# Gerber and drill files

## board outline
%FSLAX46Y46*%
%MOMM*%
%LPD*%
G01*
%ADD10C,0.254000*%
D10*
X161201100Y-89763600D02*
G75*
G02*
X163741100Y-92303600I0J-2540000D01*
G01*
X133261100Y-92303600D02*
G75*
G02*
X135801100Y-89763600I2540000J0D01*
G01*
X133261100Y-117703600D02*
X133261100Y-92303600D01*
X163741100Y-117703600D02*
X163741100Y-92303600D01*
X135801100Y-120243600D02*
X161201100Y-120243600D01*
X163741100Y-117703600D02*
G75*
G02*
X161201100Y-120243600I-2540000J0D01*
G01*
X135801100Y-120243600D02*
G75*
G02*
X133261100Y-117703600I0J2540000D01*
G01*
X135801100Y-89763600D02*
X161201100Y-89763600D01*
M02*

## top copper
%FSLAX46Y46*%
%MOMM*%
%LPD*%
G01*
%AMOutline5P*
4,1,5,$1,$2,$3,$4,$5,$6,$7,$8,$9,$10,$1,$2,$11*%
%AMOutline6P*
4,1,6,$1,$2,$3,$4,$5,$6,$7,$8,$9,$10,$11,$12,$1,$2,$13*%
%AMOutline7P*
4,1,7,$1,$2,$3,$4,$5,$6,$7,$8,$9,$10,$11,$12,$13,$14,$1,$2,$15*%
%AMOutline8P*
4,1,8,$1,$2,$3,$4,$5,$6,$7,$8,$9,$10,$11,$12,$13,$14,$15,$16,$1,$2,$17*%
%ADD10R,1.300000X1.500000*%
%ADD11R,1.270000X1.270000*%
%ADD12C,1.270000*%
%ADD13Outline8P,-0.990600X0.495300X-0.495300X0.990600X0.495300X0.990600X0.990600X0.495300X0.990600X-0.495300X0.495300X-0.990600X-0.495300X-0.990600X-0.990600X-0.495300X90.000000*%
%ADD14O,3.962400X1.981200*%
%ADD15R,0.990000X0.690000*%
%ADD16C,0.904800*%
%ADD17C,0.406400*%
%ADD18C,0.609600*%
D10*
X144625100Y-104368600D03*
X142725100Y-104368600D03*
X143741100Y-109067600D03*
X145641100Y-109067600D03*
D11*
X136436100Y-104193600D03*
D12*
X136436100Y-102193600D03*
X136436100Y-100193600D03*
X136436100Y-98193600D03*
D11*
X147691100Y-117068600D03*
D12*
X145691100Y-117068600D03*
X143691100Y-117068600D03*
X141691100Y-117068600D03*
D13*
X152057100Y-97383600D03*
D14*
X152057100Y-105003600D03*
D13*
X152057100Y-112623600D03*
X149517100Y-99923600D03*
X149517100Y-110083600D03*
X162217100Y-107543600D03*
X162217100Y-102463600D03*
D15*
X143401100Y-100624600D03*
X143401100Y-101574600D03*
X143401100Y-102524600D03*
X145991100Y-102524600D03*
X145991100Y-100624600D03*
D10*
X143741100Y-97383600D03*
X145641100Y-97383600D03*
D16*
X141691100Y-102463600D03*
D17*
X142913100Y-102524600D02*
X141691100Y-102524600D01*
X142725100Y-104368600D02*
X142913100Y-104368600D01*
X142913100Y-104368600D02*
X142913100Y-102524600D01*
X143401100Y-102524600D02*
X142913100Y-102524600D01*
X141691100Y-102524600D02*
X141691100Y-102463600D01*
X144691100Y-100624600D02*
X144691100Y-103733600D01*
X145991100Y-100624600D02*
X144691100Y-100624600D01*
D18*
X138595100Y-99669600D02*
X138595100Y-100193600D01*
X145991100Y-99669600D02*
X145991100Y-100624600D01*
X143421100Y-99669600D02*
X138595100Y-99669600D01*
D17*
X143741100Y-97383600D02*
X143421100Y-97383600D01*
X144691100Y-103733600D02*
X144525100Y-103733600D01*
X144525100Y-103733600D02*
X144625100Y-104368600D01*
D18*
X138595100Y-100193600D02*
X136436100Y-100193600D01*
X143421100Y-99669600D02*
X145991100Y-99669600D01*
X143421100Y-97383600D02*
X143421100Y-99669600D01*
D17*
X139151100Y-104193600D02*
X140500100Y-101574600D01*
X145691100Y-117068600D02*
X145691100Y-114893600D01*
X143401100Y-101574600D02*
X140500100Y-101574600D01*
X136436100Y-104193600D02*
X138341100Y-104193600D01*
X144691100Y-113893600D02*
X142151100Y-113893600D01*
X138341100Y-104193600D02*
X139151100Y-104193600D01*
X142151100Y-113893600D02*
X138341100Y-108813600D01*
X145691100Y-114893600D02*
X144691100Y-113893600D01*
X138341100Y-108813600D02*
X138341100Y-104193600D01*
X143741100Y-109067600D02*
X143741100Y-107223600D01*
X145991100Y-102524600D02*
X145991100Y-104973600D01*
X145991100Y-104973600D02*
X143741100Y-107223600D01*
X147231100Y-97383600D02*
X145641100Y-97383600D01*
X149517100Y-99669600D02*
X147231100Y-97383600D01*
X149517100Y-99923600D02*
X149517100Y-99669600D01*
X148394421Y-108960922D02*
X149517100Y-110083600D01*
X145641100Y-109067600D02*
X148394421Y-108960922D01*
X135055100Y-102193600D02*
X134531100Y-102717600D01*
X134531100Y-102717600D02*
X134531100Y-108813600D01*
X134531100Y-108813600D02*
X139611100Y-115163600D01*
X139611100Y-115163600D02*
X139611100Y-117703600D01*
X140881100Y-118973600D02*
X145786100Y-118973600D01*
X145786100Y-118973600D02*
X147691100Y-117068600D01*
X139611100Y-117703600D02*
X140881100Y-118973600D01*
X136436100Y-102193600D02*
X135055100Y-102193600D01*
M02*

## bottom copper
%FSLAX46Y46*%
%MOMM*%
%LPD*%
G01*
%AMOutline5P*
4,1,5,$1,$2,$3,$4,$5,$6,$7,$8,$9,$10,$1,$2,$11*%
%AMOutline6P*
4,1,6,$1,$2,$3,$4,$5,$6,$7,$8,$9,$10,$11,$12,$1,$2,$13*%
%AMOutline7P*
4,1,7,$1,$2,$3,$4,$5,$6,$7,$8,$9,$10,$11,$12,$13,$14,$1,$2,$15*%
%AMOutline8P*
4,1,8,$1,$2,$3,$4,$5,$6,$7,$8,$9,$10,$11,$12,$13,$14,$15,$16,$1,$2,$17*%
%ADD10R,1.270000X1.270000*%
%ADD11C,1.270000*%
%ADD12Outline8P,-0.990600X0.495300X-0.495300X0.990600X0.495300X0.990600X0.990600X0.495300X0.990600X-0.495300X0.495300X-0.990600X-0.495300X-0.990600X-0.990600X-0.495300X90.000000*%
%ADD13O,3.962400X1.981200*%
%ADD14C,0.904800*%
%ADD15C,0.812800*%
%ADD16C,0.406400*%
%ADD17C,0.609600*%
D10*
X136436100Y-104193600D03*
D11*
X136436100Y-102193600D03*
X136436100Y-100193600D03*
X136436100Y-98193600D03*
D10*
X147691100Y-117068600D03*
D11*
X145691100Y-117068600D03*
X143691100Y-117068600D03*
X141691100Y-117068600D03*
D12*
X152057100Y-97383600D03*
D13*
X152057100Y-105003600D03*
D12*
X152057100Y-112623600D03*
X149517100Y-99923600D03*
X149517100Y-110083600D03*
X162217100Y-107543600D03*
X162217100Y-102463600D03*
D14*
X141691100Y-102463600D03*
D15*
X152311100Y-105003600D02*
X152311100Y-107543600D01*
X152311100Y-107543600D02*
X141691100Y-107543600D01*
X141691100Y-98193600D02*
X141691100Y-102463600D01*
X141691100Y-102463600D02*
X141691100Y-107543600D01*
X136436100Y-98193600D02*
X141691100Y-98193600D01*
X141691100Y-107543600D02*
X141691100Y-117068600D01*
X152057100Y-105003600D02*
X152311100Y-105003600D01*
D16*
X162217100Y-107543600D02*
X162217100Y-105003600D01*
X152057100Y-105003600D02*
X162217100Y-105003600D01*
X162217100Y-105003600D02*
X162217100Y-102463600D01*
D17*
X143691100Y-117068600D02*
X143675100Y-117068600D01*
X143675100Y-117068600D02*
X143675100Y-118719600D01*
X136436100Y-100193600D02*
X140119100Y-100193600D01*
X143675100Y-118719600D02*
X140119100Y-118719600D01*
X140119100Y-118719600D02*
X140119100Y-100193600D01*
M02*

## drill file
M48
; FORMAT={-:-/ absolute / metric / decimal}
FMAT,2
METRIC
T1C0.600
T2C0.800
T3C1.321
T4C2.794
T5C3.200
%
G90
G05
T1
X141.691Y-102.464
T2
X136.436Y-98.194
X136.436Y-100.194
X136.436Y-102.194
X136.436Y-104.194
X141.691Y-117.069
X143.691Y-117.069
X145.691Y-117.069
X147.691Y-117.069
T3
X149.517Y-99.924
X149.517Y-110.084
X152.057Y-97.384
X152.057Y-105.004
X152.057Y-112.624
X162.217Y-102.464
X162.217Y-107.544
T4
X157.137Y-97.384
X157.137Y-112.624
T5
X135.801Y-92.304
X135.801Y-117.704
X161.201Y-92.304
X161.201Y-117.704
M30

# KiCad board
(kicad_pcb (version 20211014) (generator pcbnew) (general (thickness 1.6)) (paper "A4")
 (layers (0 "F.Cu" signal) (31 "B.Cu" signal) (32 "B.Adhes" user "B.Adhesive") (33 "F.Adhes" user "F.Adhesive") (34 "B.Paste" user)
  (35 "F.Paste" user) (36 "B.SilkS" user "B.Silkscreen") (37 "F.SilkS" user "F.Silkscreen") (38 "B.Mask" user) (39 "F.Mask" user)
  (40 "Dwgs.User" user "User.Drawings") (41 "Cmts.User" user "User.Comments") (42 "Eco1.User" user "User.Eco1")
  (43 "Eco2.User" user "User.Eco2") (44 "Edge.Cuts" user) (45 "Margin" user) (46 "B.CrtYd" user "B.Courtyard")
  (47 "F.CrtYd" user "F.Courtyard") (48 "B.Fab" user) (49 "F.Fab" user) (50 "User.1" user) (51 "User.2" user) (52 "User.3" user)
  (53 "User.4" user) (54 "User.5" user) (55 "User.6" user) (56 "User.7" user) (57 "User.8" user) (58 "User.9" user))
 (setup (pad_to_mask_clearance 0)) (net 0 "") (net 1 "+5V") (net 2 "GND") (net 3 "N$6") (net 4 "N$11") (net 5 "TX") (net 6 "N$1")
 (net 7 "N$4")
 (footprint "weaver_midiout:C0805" (layer "F.Cu") (at 143.6751 104.3686 180)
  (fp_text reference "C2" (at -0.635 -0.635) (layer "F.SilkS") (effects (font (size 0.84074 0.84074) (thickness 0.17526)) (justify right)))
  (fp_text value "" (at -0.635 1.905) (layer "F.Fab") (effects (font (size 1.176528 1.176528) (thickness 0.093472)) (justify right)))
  (pad "1" smd rect (at -0.95 0 180) (size 1.3 1.5) (layers "F.Cu" "F.Paste" "F.Mask") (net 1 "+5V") (solder_mask_margin 0.0508))
  (pad "2" smd rect (at 0.95 0 180) (size 1.3 1.5) (layers "F.Cu" "F.Paste" "F.Mask") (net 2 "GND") (solder_mask_margin 0.0508)))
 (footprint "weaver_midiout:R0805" (layer "F.Cu") (at 144.6911 109.0676)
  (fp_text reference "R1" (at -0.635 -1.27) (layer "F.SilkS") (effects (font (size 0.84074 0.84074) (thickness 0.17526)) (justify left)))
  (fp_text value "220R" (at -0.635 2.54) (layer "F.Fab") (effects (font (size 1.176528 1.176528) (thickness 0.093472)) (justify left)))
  (pad "1" smd rect (at -0.95 0) (size 1.3 1.5) (layers "F.Cu" "F.Paste" "F.Mask") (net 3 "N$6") (solder_mask_margin 0.0508))
  (pad "2" smd rect (at 0.95 0) (size 1.3 1.5) (layers "F.Cu" "F.Paste" "F.Mask") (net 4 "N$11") (solder_mask_margin 0.0508)))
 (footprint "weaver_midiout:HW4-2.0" (layer "F.Cu") (at 136.4361 101.1936 90)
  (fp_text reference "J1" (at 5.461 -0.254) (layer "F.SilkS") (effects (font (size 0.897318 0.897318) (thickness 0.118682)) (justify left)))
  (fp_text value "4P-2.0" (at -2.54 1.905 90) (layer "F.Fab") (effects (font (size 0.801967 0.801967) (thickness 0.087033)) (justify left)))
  (pad "1" thru_hole rect (at -3 0 90) (size 1.27 1.27) (drill 0.8) (layers *.Cu *.Mask) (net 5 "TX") (solder_mask_margin 0.0508))
  (pad "2" thru_hole circle (at -1 0 90) (size 1.27 1.27) (drill 0.8) (layers *.Cu *.Mask) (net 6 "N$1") (solder_mask_margin 0.0508))
  (pad "3" thru_hole circle (at 1 0 90) (size 1.27 1.27) (drill 0.8) (layers *.Cu *.Mask) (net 1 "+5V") (solder_mask_margin 0.0508))
  (pad "4" thru_hole circle (at 3 0 90) (size 1.27 1.27) (drill 0.8) (layers *.Cu *.Mask) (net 2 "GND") (solder_mask_margin 0.0508)))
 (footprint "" (layer "F.Cu") (at 161.2011 92.3036)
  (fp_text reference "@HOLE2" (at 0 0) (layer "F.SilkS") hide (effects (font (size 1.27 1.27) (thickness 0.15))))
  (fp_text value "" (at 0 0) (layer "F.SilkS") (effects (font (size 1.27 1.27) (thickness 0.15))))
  (pad "" np_thru_hole circle (at 0 0) (size 3.2 3.2) (drill 3.2) (layers *.Cu *.Mask)))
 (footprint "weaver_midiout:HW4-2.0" (layer "F.Cu") (at 144.6911 117.0686 180)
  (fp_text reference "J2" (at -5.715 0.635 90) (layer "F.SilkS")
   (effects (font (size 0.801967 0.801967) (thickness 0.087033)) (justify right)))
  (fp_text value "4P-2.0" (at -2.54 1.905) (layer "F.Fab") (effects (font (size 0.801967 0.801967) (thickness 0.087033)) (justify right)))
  (pad "1" thru_hole rect (at -3 0 180) (size 1.27 1.27) (drill 0.8) (layers *.Cu *.Mask) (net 6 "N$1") (solder_mask_margin 0.0508))
  (pad "2" thru_hole circle (at -1 0 180) (size 1.27 1.27) (drill 0.8) (layers *.Cu *.Mask) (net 5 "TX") (solder_mask_margin 0.0508))
  (pad "3" thru_hole circle (at 1 0 180) (size 1.27 1.27) (drill 0.8) (layers *.Cu *.Mask) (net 1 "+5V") (solder_mask_margin 0.0508))
  (pad "4" thru_hole circle (at 3 0 180) (size 1.27 1.27) (drill 0.8) (layers *.Cu *.Mask) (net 2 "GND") (solder_mask_margin 0.0508)))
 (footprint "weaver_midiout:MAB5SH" (layer "F.Cu") (at 157.1371 105.0036 90)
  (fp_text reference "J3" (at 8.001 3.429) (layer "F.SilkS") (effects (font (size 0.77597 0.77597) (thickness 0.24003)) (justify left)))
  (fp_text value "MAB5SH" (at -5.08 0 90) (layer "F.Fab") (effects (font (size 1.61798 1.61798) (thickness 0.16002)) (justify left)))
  (pad "" np_thru_hole circle (at -7.62 0 90) (size 2.794 2.794) (drill 2.794) (layers *.Cu *.Mask))
  (pad "" np_thru_hole circle (at 7.62 0 90) (size 2.794 2.794) (drill 2.794) (layers *.Cu *.Mask))
  (pad "1" thru_hole roundrect (at 7.62 -5.08 90) (size 1.9812 1.9812) (drill 1.3208) (layers *.Cu *.Mask) (roundrect_rratio 0.25)
   (chamfer_ratio 0.25) (chamfer top_left top_right bottom_left bottom_right) (solder_mask_margin 0.0508))
  (pad "2" thru_hole oval (at 0 -5.08 180) (size 3.9624 1.9812) (drill 1.3208) (layers *.Cu *.Mask) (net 2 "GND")
   (solder_mask_margin 0.0508))
  (pad "3" thru_hole roundrect (at -7.62 -5.08 90) (size 1.9812 1.9812) (drill 1.3208) (layers *.Cu *.Mask) (roundrect_rratio 0.25)
   (chamfer_ratio 0.25) (chamfer top_left top_right bottom_left bottom_right) (solder_mask_margin 0.0508))
  (pad "4" thru_hole roundrect (at 5.08 -7.62 90) (size 1.9812 1.9812) (drill 1.3208) (layers *.Cu *.Mask) (roundrect_rratio 0.25)
   (chamfer_ratio 0.25) (chamfer top_left top_right bottom_left bottom_right) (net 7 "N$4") (solder_mask_margin 0.0508))
  (pad "5" thru_hole roundrect (at -5.08 -7.62 90) (size 1.9812 1.9812) (drill 1.3208) (layers *.Cu *.Mask) (roundrect_rratio 0.25)
   (chamfer_ratio 0.25) (chamfer top_left top_right bottom_left bottom_right) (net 4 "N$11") (solder_mask_margin 0.0508))
  (pad "PE" thru_hole roundrect (at -2.54 5.08 90) (size 1.9812 1.9812) (drill 1.3208) (layers *.Cu *.Mask) (roundrect_rratio 0.25)
   (chamfer_ratio 0.25) (chamfer top_left top_right bottom_left bottom_right) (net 2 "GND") (solder_mask_margin 0.0508))
  (pad "PE@" thru_hole roundrect (at 2.54 5.08 90) (size 1.9812 1.9812) (drill 1.3208) (layers *.Cu *.Mask) (roundrect_rratio 0.25)
   (chamfer_ratio 0.25) (chamfer top_left top_right bottom_left bottom_right) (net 2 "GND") (solder_mask_margin 0.0508)))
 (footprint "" (layer "F.Cu") (at 161.2011 117.7036)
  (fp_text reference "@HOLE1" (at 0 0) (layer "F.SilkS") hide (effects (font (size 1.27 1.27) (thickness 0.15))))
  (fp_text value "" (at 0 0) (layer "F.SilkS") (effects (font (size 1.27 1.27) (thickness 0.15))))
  (pad "" np_thru_hole circle (at 0 0) (size 3.2 3.2) (drill 3.2) (layers *.Cu *.Mask)))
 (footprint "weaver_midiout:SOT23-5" (layer "F.Cu") (at 144.6911 101.5746 -90)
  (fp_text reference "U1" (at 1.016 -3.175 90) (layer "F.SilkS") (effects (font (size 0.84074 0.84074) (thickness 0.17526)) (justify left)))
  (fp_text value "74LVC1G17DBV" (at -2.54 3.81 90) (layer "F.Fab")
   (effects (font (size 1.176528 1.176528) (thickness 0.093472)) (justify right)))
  (pad "1" smd rect (at -0.95 1.29 270) (size 0.69 0.99) (layers "F.Cu" "F.Paste" "F.Mask") (solder_mask_margin 0.0508))
  (pad "2" smd rect (at 0 1.29 270) (size 0.69 0.99) (layers "F.Cu" "F.Paste" "F.Mask") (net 5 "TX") (solder_mask_margin 0.0508))
  (pad "3" smd rect (at 0.95 1.29 270) (size 0.69 0.99) (layers "F.Cu" "F.Paste" "F.Mask") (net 2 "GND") (solder_mask_margin 0.0508))
  (pad "4" smd rect (at 0.95 -1.3 270) (size 0.69 0.99) (layers "F.Cu" "F.Paste" "F.Mask") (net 3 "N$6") (solder_mask_margin 0.0508))
  (pad "5" smd rect (at -0.95 -1.3 270) (size 0.69 0.99) (layers "F.Cu" "F.Paste" "F.Mask") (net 1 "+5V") (solder_mask_margin 0.0508)))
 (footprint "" (layer "F.Cu") (at 135.8011 117.7036)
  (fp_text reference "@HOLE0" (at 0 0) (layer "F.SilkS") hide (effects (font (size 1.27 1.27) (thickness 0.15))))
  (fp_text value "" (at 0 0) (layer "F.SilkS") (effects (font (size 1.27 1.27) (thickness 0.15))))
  (pad "" np_thru_hole circle (at 0 0) (size 3.2 3.2) (drill 3.2) (layers *.Cu *.Mask)))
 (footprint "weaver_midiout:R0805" (layer "F.Cu") (at 144.6911 97.3836)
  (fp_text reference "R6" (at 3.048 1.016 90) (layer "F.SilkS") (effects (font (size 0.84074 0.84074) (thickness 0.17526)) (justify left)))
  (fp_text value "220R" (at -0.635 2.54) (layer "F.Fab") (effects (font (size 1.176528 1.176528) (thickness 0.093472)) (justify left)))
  (pad "1" smd rect (at -0.95 0) (size 1.3 1.5) (layers "F.Cu" "F.Paste" "F.Mask") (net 1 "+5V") (solder_mask_margin 0.0508))
  (pad "2" smd rect (at 0.95 0) (size 1.3 1.5) (layers "F.Cu" "F.Paste" "F.Mask") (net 7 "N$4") (solder_mask_margin 0.0508)))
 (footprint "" (layer "F.Cu") (at 135.8011 92.3036)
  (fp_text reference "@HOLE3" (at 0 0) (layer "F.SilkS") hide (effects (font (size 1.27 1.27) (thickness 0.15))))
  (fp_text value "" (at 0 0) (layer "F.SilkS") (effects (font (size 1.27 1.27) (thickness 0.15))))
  (pad "" np_thru_hole circle (at 0 0) (size 3.2 3.2) (drill 3.2) (layers *.Cu *.Mask)))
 (gr_arc (start 161.2011 89.7636) (mid 162.997151 90.507549) (end 163.7411 92.3036) (layer "Edge.Cuts") (width 0.254))
 (gr_arc (start 133.2611 92.3036) (mid 134.005049 90.507549) (end 135.8011 89.7636) (layer "Edge.Cuts") (width 0.254))
 (gr_line (start 133.2611 117.7036) (end 133.2611 92.3036) (layer "Edge.Cuts") (width 0.254))
 (gr_line (start 163.7411 117.7036) (end 163.7411 92.3036) (layer "Edge.Cuts") (width 0.254))
 (gr_line (start 135.8011 120.2436) (end 161.2011 120.2436) (layer "Edge.Cuts") (width 0.254))
 (gr_arc (start 163.7411 117.7036) (mid 162.997151 119.499651) (end 161.2011 120.2436) (layer "Edge.Cuts") (width 0.254))
 (gr_arc (start 135.8011 120.2436) (mid 134.005049 119.499651) (end 133.2611 117.7036) (layer "Edge.Cuts") (width 0.254))
 (gr_line (start 135.8011 89.7636) (end 161.2011 89.7636) (layer "Edge.Cuts") (width 0.254))
 (segment (start 142.9131 102.5246) (end 141.6911 102.5246) (width 0.4064) (layer "F.Cu") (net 2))
 (segment (start 142.7251 104.3686) (end 142.9131 104.3686) (width 0.4064) (layer "F.Cu") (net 2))
 (segment (start 142.9131 104.3686) (end 142.9131 102.5246) (width 0.4064) (layer "F.Cu") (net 2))
 (segment (start 143.4011 102.5246) (end 142.9131 102.5246) (width 0.4064) (layer "F.Cu") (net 2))
 (segment (start 141.6911 102.5246) (end 141.6911 102.4636) (width 0.4064) (layer "F.Cu") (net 2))
 (via (at 141.6911 102.4636) (size 0.9048) (drill 0.6) (layers "F.Cu" "B.Cu") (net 2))
 (segment (start 152.3111 105.0036) (end 152.3111 107.5436) (width 0.8128) (layer "B.Cu") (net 2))
 (segment (start 152.3111 107.5436) (end 141.6911 107.5436) (width 0.8128) (layer "B.Cu") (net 2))
 (segment (start 141.6911 98.1936) (end 141.6911 102.4636) (width 0.8128) (layer "B.Cu") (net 2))
 (segment (start 141.6911 102.4636) (end 141.6911 107.5436) (width 0.8128) (layer "B.Cu") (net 2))
 (segment (start 136.4361 98.1936) (end 141.6911 98.1936) (width 0.8128) (layer "B.Cu") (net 2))
 (segment (start 141.6911 107.5436) (end 141.6911 117.0686) (width 0.8128) (layer "B.Cu") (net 2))
 (segment (start 152.0571 105.0036) (end 152.3111 105.0036) (width 0.8128) (layer "B.Cu") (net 2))
 (segment (start 162.2171 107.5436) (end 162.2171 105.0036) (width 0.4064) (layer "B.Cu") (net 2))
 (segment (start 152.0571 105.0036) (end 162.2171 105.0036) (width 0.4064) (layer "B.Cu") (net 2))
 (segment (start 162.2171 105.0036) (end 162.2171 102.4636) (width 0.4064) (layer "B.Cu") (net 2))
 (segment (start 144.6911 100.6246) (end 144.6911 103.7336) (width 0.4064) (layer "F.Cu") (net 1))
 (segment (start 145.9911 100.6246) (end 144.6911 100.6246) (width 0.4064) (layer "F.Cu") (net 1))
 (segment (start 138.5951 99.6696) (end 138.5951 100.1936) (width 0.6096) (layer "F.Cu") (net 1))
 (segment (start 145.9911 99.6696) (end 145.9911 100.6246) (width 0.6096) (layer "F.Cu") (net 1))
 (segment (start 143.4211 99.6696) (end 138.5951 99.6696) (width 0.6096) (layer "F.Cu") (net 1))
 (segment (start 143.7411 97.3836) (end 143.4211 97.3836) (width 0.4064) (layer "F.Cu") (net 1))
 (segment (start 144.6911 103.7336) (end 144.5251 103.7336) (width 0.4064) (layer "F.Cu") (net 1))
 (segment (start 144.5251 103.7336) (end 144.6251 104.3686) (width 0.4064) (layer "F.Cu") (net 1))
 (segment (start 138.5951 100.1936) (end 136.4361 100.1936) (width 0.6096) (layer "F.Cu") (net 1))
 (segment (start 143.4211 99.6696) (end 145.9911 99.6696) (width 0.6096) (layer "F.Cu") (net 1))
 (segment (start 143.4211 97.3836) (end 143.4211 99.6696) (width 0.6096) (layer "F.Cu") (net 1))
 (segment (start 143.6911 117.0686) (end 143.6751 117.0686) (width 0.6096) (layer "B.Cu") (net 1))
 (segment (start 143.6751 117.0686) (end 143.6751 118.7196) (width 0.6096) (layer "B.Cu") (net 1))
 (segment (start 136.4361 100.1936) (end 140.1191 100.1936) (width 0.6096) (layer "B.Cu") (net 1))
 (segment (start 143.6751 118.7196) (end 140.1191 118.7196) (width 0.6096) (layer "B.Cu") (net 1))
 (segment (start 140.1191 118.7196) (end 140.1191 100.1936) (width 0.6096) (layer "B.Cu") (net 1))
 (segment (start 139.1511 104.1936) (end 140.5001 101.5746) (width 0.4064) (layer "F.Cu") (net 5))
 (segment (start 145.6911 117.0686) (end 145.6911 114.8936) (width 0.4064) (layer "F.Cu") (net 5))
 (segment (start 143.4011 101.5746) (end 140.5001 101.5746) (width 0.4064) (layer "F.Cu") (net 5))
 (segment (start 136.4361 104.1936) (end 138.3411 104.1936) (width 0.4064) (layer "F.Cu") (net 5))
 (segment (start 144.6911 113.8936) (end 142.1511 113.8936) (width 0.4064) (layer "F.Cu") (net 5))
 (segment (start 138.3411 104.1936) (end 139.1511 104.1936) (width 0.4064) (layer "F.Cu") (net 5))
 (segment (start 142.1511 113.8936) (end 138.3411 108.8136) (width 0.4064) (layer "F.Cu") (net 5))
 (segment (start 145.6911 114.8936) (end 144.6911 113.8936) (width 0.4064) (layer "F.Cu") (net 5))
 (segment (start 138.3411 108.8136) (end 138.3411 104.1936) (width 0.4064) (layer "F.Cu") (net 5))
 (segment (start 143.7411 109.0676) (end 143.7411 107.2236) (width 0.4064) (layer "F.Cu") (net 3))
 (segment (start 145.9911 102.5246) (end 145.9911 104.9736) (width 0.4064) (layer "F.Cu") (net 3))
 (segment (start 145.9911 104.9736) (end 143.7411 107.2236) (width 0.4064) (layer "F.Cu") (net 3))
 (segment (start 147.2311 97.3836) (end 145.6411 97.3836) (width 0.4064) (layer "F.Cu") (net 7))
 (segment (start 149.5171 99.6696) (end 147.2311 97.3836) (width 0.4064) (layer "F.Cu") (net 7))
 (segment (start 149.5171 99.9236) (end 149.5171 99.6696) (width 0.4064) (layer "F.Cu") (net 7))
 (segment (start 148.394421 108.960922) (end 149.5171 110.0836) (width 0.4064) (layer "F.Cu") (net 4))
 (segment (start 145.6411 109.0676) (end 148.394421 108.960922) (width 0.4064) (layer "F.Cu") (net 4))
 (segment (start 135.0551 102.1936) (end 134.5311 102.7176) (width 0.4064) (layer "F.Cu") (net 6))
 (segment (start 134.5311 102.7176) (end 134.5311 108.8136) (width 0.4064) (layer "F.Cu") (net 6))
 (segment (start 134.5311 108.8136) (end 139.6111 115.1636) (width 0.4064) (layer "F.Cu") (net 6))
 (segment (start 139.6111 115.1636) (end 139.6111 117.7036) (width 0.4064) (layer "F.Cu") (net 6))
 (segment (start 140.8811 118.9736) (end 145.7861 118.9736) (width 0.4064) (layer "F.Cu") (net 6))
 (segment (start 145.7861 118.9736) (end 147.6911 117.0686) (width 0.4064) (layer "F.Cu") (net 6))
 (segment (start 139.6111 117.7036) (end 140.8811 118.9736) (width 0.4064) (layer "F.Cu") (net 6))
 (segment (start 136.4361 102.1936) (end 135.0551 102.1936) (width 0.4064) (layer "F.Cu") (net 6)))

